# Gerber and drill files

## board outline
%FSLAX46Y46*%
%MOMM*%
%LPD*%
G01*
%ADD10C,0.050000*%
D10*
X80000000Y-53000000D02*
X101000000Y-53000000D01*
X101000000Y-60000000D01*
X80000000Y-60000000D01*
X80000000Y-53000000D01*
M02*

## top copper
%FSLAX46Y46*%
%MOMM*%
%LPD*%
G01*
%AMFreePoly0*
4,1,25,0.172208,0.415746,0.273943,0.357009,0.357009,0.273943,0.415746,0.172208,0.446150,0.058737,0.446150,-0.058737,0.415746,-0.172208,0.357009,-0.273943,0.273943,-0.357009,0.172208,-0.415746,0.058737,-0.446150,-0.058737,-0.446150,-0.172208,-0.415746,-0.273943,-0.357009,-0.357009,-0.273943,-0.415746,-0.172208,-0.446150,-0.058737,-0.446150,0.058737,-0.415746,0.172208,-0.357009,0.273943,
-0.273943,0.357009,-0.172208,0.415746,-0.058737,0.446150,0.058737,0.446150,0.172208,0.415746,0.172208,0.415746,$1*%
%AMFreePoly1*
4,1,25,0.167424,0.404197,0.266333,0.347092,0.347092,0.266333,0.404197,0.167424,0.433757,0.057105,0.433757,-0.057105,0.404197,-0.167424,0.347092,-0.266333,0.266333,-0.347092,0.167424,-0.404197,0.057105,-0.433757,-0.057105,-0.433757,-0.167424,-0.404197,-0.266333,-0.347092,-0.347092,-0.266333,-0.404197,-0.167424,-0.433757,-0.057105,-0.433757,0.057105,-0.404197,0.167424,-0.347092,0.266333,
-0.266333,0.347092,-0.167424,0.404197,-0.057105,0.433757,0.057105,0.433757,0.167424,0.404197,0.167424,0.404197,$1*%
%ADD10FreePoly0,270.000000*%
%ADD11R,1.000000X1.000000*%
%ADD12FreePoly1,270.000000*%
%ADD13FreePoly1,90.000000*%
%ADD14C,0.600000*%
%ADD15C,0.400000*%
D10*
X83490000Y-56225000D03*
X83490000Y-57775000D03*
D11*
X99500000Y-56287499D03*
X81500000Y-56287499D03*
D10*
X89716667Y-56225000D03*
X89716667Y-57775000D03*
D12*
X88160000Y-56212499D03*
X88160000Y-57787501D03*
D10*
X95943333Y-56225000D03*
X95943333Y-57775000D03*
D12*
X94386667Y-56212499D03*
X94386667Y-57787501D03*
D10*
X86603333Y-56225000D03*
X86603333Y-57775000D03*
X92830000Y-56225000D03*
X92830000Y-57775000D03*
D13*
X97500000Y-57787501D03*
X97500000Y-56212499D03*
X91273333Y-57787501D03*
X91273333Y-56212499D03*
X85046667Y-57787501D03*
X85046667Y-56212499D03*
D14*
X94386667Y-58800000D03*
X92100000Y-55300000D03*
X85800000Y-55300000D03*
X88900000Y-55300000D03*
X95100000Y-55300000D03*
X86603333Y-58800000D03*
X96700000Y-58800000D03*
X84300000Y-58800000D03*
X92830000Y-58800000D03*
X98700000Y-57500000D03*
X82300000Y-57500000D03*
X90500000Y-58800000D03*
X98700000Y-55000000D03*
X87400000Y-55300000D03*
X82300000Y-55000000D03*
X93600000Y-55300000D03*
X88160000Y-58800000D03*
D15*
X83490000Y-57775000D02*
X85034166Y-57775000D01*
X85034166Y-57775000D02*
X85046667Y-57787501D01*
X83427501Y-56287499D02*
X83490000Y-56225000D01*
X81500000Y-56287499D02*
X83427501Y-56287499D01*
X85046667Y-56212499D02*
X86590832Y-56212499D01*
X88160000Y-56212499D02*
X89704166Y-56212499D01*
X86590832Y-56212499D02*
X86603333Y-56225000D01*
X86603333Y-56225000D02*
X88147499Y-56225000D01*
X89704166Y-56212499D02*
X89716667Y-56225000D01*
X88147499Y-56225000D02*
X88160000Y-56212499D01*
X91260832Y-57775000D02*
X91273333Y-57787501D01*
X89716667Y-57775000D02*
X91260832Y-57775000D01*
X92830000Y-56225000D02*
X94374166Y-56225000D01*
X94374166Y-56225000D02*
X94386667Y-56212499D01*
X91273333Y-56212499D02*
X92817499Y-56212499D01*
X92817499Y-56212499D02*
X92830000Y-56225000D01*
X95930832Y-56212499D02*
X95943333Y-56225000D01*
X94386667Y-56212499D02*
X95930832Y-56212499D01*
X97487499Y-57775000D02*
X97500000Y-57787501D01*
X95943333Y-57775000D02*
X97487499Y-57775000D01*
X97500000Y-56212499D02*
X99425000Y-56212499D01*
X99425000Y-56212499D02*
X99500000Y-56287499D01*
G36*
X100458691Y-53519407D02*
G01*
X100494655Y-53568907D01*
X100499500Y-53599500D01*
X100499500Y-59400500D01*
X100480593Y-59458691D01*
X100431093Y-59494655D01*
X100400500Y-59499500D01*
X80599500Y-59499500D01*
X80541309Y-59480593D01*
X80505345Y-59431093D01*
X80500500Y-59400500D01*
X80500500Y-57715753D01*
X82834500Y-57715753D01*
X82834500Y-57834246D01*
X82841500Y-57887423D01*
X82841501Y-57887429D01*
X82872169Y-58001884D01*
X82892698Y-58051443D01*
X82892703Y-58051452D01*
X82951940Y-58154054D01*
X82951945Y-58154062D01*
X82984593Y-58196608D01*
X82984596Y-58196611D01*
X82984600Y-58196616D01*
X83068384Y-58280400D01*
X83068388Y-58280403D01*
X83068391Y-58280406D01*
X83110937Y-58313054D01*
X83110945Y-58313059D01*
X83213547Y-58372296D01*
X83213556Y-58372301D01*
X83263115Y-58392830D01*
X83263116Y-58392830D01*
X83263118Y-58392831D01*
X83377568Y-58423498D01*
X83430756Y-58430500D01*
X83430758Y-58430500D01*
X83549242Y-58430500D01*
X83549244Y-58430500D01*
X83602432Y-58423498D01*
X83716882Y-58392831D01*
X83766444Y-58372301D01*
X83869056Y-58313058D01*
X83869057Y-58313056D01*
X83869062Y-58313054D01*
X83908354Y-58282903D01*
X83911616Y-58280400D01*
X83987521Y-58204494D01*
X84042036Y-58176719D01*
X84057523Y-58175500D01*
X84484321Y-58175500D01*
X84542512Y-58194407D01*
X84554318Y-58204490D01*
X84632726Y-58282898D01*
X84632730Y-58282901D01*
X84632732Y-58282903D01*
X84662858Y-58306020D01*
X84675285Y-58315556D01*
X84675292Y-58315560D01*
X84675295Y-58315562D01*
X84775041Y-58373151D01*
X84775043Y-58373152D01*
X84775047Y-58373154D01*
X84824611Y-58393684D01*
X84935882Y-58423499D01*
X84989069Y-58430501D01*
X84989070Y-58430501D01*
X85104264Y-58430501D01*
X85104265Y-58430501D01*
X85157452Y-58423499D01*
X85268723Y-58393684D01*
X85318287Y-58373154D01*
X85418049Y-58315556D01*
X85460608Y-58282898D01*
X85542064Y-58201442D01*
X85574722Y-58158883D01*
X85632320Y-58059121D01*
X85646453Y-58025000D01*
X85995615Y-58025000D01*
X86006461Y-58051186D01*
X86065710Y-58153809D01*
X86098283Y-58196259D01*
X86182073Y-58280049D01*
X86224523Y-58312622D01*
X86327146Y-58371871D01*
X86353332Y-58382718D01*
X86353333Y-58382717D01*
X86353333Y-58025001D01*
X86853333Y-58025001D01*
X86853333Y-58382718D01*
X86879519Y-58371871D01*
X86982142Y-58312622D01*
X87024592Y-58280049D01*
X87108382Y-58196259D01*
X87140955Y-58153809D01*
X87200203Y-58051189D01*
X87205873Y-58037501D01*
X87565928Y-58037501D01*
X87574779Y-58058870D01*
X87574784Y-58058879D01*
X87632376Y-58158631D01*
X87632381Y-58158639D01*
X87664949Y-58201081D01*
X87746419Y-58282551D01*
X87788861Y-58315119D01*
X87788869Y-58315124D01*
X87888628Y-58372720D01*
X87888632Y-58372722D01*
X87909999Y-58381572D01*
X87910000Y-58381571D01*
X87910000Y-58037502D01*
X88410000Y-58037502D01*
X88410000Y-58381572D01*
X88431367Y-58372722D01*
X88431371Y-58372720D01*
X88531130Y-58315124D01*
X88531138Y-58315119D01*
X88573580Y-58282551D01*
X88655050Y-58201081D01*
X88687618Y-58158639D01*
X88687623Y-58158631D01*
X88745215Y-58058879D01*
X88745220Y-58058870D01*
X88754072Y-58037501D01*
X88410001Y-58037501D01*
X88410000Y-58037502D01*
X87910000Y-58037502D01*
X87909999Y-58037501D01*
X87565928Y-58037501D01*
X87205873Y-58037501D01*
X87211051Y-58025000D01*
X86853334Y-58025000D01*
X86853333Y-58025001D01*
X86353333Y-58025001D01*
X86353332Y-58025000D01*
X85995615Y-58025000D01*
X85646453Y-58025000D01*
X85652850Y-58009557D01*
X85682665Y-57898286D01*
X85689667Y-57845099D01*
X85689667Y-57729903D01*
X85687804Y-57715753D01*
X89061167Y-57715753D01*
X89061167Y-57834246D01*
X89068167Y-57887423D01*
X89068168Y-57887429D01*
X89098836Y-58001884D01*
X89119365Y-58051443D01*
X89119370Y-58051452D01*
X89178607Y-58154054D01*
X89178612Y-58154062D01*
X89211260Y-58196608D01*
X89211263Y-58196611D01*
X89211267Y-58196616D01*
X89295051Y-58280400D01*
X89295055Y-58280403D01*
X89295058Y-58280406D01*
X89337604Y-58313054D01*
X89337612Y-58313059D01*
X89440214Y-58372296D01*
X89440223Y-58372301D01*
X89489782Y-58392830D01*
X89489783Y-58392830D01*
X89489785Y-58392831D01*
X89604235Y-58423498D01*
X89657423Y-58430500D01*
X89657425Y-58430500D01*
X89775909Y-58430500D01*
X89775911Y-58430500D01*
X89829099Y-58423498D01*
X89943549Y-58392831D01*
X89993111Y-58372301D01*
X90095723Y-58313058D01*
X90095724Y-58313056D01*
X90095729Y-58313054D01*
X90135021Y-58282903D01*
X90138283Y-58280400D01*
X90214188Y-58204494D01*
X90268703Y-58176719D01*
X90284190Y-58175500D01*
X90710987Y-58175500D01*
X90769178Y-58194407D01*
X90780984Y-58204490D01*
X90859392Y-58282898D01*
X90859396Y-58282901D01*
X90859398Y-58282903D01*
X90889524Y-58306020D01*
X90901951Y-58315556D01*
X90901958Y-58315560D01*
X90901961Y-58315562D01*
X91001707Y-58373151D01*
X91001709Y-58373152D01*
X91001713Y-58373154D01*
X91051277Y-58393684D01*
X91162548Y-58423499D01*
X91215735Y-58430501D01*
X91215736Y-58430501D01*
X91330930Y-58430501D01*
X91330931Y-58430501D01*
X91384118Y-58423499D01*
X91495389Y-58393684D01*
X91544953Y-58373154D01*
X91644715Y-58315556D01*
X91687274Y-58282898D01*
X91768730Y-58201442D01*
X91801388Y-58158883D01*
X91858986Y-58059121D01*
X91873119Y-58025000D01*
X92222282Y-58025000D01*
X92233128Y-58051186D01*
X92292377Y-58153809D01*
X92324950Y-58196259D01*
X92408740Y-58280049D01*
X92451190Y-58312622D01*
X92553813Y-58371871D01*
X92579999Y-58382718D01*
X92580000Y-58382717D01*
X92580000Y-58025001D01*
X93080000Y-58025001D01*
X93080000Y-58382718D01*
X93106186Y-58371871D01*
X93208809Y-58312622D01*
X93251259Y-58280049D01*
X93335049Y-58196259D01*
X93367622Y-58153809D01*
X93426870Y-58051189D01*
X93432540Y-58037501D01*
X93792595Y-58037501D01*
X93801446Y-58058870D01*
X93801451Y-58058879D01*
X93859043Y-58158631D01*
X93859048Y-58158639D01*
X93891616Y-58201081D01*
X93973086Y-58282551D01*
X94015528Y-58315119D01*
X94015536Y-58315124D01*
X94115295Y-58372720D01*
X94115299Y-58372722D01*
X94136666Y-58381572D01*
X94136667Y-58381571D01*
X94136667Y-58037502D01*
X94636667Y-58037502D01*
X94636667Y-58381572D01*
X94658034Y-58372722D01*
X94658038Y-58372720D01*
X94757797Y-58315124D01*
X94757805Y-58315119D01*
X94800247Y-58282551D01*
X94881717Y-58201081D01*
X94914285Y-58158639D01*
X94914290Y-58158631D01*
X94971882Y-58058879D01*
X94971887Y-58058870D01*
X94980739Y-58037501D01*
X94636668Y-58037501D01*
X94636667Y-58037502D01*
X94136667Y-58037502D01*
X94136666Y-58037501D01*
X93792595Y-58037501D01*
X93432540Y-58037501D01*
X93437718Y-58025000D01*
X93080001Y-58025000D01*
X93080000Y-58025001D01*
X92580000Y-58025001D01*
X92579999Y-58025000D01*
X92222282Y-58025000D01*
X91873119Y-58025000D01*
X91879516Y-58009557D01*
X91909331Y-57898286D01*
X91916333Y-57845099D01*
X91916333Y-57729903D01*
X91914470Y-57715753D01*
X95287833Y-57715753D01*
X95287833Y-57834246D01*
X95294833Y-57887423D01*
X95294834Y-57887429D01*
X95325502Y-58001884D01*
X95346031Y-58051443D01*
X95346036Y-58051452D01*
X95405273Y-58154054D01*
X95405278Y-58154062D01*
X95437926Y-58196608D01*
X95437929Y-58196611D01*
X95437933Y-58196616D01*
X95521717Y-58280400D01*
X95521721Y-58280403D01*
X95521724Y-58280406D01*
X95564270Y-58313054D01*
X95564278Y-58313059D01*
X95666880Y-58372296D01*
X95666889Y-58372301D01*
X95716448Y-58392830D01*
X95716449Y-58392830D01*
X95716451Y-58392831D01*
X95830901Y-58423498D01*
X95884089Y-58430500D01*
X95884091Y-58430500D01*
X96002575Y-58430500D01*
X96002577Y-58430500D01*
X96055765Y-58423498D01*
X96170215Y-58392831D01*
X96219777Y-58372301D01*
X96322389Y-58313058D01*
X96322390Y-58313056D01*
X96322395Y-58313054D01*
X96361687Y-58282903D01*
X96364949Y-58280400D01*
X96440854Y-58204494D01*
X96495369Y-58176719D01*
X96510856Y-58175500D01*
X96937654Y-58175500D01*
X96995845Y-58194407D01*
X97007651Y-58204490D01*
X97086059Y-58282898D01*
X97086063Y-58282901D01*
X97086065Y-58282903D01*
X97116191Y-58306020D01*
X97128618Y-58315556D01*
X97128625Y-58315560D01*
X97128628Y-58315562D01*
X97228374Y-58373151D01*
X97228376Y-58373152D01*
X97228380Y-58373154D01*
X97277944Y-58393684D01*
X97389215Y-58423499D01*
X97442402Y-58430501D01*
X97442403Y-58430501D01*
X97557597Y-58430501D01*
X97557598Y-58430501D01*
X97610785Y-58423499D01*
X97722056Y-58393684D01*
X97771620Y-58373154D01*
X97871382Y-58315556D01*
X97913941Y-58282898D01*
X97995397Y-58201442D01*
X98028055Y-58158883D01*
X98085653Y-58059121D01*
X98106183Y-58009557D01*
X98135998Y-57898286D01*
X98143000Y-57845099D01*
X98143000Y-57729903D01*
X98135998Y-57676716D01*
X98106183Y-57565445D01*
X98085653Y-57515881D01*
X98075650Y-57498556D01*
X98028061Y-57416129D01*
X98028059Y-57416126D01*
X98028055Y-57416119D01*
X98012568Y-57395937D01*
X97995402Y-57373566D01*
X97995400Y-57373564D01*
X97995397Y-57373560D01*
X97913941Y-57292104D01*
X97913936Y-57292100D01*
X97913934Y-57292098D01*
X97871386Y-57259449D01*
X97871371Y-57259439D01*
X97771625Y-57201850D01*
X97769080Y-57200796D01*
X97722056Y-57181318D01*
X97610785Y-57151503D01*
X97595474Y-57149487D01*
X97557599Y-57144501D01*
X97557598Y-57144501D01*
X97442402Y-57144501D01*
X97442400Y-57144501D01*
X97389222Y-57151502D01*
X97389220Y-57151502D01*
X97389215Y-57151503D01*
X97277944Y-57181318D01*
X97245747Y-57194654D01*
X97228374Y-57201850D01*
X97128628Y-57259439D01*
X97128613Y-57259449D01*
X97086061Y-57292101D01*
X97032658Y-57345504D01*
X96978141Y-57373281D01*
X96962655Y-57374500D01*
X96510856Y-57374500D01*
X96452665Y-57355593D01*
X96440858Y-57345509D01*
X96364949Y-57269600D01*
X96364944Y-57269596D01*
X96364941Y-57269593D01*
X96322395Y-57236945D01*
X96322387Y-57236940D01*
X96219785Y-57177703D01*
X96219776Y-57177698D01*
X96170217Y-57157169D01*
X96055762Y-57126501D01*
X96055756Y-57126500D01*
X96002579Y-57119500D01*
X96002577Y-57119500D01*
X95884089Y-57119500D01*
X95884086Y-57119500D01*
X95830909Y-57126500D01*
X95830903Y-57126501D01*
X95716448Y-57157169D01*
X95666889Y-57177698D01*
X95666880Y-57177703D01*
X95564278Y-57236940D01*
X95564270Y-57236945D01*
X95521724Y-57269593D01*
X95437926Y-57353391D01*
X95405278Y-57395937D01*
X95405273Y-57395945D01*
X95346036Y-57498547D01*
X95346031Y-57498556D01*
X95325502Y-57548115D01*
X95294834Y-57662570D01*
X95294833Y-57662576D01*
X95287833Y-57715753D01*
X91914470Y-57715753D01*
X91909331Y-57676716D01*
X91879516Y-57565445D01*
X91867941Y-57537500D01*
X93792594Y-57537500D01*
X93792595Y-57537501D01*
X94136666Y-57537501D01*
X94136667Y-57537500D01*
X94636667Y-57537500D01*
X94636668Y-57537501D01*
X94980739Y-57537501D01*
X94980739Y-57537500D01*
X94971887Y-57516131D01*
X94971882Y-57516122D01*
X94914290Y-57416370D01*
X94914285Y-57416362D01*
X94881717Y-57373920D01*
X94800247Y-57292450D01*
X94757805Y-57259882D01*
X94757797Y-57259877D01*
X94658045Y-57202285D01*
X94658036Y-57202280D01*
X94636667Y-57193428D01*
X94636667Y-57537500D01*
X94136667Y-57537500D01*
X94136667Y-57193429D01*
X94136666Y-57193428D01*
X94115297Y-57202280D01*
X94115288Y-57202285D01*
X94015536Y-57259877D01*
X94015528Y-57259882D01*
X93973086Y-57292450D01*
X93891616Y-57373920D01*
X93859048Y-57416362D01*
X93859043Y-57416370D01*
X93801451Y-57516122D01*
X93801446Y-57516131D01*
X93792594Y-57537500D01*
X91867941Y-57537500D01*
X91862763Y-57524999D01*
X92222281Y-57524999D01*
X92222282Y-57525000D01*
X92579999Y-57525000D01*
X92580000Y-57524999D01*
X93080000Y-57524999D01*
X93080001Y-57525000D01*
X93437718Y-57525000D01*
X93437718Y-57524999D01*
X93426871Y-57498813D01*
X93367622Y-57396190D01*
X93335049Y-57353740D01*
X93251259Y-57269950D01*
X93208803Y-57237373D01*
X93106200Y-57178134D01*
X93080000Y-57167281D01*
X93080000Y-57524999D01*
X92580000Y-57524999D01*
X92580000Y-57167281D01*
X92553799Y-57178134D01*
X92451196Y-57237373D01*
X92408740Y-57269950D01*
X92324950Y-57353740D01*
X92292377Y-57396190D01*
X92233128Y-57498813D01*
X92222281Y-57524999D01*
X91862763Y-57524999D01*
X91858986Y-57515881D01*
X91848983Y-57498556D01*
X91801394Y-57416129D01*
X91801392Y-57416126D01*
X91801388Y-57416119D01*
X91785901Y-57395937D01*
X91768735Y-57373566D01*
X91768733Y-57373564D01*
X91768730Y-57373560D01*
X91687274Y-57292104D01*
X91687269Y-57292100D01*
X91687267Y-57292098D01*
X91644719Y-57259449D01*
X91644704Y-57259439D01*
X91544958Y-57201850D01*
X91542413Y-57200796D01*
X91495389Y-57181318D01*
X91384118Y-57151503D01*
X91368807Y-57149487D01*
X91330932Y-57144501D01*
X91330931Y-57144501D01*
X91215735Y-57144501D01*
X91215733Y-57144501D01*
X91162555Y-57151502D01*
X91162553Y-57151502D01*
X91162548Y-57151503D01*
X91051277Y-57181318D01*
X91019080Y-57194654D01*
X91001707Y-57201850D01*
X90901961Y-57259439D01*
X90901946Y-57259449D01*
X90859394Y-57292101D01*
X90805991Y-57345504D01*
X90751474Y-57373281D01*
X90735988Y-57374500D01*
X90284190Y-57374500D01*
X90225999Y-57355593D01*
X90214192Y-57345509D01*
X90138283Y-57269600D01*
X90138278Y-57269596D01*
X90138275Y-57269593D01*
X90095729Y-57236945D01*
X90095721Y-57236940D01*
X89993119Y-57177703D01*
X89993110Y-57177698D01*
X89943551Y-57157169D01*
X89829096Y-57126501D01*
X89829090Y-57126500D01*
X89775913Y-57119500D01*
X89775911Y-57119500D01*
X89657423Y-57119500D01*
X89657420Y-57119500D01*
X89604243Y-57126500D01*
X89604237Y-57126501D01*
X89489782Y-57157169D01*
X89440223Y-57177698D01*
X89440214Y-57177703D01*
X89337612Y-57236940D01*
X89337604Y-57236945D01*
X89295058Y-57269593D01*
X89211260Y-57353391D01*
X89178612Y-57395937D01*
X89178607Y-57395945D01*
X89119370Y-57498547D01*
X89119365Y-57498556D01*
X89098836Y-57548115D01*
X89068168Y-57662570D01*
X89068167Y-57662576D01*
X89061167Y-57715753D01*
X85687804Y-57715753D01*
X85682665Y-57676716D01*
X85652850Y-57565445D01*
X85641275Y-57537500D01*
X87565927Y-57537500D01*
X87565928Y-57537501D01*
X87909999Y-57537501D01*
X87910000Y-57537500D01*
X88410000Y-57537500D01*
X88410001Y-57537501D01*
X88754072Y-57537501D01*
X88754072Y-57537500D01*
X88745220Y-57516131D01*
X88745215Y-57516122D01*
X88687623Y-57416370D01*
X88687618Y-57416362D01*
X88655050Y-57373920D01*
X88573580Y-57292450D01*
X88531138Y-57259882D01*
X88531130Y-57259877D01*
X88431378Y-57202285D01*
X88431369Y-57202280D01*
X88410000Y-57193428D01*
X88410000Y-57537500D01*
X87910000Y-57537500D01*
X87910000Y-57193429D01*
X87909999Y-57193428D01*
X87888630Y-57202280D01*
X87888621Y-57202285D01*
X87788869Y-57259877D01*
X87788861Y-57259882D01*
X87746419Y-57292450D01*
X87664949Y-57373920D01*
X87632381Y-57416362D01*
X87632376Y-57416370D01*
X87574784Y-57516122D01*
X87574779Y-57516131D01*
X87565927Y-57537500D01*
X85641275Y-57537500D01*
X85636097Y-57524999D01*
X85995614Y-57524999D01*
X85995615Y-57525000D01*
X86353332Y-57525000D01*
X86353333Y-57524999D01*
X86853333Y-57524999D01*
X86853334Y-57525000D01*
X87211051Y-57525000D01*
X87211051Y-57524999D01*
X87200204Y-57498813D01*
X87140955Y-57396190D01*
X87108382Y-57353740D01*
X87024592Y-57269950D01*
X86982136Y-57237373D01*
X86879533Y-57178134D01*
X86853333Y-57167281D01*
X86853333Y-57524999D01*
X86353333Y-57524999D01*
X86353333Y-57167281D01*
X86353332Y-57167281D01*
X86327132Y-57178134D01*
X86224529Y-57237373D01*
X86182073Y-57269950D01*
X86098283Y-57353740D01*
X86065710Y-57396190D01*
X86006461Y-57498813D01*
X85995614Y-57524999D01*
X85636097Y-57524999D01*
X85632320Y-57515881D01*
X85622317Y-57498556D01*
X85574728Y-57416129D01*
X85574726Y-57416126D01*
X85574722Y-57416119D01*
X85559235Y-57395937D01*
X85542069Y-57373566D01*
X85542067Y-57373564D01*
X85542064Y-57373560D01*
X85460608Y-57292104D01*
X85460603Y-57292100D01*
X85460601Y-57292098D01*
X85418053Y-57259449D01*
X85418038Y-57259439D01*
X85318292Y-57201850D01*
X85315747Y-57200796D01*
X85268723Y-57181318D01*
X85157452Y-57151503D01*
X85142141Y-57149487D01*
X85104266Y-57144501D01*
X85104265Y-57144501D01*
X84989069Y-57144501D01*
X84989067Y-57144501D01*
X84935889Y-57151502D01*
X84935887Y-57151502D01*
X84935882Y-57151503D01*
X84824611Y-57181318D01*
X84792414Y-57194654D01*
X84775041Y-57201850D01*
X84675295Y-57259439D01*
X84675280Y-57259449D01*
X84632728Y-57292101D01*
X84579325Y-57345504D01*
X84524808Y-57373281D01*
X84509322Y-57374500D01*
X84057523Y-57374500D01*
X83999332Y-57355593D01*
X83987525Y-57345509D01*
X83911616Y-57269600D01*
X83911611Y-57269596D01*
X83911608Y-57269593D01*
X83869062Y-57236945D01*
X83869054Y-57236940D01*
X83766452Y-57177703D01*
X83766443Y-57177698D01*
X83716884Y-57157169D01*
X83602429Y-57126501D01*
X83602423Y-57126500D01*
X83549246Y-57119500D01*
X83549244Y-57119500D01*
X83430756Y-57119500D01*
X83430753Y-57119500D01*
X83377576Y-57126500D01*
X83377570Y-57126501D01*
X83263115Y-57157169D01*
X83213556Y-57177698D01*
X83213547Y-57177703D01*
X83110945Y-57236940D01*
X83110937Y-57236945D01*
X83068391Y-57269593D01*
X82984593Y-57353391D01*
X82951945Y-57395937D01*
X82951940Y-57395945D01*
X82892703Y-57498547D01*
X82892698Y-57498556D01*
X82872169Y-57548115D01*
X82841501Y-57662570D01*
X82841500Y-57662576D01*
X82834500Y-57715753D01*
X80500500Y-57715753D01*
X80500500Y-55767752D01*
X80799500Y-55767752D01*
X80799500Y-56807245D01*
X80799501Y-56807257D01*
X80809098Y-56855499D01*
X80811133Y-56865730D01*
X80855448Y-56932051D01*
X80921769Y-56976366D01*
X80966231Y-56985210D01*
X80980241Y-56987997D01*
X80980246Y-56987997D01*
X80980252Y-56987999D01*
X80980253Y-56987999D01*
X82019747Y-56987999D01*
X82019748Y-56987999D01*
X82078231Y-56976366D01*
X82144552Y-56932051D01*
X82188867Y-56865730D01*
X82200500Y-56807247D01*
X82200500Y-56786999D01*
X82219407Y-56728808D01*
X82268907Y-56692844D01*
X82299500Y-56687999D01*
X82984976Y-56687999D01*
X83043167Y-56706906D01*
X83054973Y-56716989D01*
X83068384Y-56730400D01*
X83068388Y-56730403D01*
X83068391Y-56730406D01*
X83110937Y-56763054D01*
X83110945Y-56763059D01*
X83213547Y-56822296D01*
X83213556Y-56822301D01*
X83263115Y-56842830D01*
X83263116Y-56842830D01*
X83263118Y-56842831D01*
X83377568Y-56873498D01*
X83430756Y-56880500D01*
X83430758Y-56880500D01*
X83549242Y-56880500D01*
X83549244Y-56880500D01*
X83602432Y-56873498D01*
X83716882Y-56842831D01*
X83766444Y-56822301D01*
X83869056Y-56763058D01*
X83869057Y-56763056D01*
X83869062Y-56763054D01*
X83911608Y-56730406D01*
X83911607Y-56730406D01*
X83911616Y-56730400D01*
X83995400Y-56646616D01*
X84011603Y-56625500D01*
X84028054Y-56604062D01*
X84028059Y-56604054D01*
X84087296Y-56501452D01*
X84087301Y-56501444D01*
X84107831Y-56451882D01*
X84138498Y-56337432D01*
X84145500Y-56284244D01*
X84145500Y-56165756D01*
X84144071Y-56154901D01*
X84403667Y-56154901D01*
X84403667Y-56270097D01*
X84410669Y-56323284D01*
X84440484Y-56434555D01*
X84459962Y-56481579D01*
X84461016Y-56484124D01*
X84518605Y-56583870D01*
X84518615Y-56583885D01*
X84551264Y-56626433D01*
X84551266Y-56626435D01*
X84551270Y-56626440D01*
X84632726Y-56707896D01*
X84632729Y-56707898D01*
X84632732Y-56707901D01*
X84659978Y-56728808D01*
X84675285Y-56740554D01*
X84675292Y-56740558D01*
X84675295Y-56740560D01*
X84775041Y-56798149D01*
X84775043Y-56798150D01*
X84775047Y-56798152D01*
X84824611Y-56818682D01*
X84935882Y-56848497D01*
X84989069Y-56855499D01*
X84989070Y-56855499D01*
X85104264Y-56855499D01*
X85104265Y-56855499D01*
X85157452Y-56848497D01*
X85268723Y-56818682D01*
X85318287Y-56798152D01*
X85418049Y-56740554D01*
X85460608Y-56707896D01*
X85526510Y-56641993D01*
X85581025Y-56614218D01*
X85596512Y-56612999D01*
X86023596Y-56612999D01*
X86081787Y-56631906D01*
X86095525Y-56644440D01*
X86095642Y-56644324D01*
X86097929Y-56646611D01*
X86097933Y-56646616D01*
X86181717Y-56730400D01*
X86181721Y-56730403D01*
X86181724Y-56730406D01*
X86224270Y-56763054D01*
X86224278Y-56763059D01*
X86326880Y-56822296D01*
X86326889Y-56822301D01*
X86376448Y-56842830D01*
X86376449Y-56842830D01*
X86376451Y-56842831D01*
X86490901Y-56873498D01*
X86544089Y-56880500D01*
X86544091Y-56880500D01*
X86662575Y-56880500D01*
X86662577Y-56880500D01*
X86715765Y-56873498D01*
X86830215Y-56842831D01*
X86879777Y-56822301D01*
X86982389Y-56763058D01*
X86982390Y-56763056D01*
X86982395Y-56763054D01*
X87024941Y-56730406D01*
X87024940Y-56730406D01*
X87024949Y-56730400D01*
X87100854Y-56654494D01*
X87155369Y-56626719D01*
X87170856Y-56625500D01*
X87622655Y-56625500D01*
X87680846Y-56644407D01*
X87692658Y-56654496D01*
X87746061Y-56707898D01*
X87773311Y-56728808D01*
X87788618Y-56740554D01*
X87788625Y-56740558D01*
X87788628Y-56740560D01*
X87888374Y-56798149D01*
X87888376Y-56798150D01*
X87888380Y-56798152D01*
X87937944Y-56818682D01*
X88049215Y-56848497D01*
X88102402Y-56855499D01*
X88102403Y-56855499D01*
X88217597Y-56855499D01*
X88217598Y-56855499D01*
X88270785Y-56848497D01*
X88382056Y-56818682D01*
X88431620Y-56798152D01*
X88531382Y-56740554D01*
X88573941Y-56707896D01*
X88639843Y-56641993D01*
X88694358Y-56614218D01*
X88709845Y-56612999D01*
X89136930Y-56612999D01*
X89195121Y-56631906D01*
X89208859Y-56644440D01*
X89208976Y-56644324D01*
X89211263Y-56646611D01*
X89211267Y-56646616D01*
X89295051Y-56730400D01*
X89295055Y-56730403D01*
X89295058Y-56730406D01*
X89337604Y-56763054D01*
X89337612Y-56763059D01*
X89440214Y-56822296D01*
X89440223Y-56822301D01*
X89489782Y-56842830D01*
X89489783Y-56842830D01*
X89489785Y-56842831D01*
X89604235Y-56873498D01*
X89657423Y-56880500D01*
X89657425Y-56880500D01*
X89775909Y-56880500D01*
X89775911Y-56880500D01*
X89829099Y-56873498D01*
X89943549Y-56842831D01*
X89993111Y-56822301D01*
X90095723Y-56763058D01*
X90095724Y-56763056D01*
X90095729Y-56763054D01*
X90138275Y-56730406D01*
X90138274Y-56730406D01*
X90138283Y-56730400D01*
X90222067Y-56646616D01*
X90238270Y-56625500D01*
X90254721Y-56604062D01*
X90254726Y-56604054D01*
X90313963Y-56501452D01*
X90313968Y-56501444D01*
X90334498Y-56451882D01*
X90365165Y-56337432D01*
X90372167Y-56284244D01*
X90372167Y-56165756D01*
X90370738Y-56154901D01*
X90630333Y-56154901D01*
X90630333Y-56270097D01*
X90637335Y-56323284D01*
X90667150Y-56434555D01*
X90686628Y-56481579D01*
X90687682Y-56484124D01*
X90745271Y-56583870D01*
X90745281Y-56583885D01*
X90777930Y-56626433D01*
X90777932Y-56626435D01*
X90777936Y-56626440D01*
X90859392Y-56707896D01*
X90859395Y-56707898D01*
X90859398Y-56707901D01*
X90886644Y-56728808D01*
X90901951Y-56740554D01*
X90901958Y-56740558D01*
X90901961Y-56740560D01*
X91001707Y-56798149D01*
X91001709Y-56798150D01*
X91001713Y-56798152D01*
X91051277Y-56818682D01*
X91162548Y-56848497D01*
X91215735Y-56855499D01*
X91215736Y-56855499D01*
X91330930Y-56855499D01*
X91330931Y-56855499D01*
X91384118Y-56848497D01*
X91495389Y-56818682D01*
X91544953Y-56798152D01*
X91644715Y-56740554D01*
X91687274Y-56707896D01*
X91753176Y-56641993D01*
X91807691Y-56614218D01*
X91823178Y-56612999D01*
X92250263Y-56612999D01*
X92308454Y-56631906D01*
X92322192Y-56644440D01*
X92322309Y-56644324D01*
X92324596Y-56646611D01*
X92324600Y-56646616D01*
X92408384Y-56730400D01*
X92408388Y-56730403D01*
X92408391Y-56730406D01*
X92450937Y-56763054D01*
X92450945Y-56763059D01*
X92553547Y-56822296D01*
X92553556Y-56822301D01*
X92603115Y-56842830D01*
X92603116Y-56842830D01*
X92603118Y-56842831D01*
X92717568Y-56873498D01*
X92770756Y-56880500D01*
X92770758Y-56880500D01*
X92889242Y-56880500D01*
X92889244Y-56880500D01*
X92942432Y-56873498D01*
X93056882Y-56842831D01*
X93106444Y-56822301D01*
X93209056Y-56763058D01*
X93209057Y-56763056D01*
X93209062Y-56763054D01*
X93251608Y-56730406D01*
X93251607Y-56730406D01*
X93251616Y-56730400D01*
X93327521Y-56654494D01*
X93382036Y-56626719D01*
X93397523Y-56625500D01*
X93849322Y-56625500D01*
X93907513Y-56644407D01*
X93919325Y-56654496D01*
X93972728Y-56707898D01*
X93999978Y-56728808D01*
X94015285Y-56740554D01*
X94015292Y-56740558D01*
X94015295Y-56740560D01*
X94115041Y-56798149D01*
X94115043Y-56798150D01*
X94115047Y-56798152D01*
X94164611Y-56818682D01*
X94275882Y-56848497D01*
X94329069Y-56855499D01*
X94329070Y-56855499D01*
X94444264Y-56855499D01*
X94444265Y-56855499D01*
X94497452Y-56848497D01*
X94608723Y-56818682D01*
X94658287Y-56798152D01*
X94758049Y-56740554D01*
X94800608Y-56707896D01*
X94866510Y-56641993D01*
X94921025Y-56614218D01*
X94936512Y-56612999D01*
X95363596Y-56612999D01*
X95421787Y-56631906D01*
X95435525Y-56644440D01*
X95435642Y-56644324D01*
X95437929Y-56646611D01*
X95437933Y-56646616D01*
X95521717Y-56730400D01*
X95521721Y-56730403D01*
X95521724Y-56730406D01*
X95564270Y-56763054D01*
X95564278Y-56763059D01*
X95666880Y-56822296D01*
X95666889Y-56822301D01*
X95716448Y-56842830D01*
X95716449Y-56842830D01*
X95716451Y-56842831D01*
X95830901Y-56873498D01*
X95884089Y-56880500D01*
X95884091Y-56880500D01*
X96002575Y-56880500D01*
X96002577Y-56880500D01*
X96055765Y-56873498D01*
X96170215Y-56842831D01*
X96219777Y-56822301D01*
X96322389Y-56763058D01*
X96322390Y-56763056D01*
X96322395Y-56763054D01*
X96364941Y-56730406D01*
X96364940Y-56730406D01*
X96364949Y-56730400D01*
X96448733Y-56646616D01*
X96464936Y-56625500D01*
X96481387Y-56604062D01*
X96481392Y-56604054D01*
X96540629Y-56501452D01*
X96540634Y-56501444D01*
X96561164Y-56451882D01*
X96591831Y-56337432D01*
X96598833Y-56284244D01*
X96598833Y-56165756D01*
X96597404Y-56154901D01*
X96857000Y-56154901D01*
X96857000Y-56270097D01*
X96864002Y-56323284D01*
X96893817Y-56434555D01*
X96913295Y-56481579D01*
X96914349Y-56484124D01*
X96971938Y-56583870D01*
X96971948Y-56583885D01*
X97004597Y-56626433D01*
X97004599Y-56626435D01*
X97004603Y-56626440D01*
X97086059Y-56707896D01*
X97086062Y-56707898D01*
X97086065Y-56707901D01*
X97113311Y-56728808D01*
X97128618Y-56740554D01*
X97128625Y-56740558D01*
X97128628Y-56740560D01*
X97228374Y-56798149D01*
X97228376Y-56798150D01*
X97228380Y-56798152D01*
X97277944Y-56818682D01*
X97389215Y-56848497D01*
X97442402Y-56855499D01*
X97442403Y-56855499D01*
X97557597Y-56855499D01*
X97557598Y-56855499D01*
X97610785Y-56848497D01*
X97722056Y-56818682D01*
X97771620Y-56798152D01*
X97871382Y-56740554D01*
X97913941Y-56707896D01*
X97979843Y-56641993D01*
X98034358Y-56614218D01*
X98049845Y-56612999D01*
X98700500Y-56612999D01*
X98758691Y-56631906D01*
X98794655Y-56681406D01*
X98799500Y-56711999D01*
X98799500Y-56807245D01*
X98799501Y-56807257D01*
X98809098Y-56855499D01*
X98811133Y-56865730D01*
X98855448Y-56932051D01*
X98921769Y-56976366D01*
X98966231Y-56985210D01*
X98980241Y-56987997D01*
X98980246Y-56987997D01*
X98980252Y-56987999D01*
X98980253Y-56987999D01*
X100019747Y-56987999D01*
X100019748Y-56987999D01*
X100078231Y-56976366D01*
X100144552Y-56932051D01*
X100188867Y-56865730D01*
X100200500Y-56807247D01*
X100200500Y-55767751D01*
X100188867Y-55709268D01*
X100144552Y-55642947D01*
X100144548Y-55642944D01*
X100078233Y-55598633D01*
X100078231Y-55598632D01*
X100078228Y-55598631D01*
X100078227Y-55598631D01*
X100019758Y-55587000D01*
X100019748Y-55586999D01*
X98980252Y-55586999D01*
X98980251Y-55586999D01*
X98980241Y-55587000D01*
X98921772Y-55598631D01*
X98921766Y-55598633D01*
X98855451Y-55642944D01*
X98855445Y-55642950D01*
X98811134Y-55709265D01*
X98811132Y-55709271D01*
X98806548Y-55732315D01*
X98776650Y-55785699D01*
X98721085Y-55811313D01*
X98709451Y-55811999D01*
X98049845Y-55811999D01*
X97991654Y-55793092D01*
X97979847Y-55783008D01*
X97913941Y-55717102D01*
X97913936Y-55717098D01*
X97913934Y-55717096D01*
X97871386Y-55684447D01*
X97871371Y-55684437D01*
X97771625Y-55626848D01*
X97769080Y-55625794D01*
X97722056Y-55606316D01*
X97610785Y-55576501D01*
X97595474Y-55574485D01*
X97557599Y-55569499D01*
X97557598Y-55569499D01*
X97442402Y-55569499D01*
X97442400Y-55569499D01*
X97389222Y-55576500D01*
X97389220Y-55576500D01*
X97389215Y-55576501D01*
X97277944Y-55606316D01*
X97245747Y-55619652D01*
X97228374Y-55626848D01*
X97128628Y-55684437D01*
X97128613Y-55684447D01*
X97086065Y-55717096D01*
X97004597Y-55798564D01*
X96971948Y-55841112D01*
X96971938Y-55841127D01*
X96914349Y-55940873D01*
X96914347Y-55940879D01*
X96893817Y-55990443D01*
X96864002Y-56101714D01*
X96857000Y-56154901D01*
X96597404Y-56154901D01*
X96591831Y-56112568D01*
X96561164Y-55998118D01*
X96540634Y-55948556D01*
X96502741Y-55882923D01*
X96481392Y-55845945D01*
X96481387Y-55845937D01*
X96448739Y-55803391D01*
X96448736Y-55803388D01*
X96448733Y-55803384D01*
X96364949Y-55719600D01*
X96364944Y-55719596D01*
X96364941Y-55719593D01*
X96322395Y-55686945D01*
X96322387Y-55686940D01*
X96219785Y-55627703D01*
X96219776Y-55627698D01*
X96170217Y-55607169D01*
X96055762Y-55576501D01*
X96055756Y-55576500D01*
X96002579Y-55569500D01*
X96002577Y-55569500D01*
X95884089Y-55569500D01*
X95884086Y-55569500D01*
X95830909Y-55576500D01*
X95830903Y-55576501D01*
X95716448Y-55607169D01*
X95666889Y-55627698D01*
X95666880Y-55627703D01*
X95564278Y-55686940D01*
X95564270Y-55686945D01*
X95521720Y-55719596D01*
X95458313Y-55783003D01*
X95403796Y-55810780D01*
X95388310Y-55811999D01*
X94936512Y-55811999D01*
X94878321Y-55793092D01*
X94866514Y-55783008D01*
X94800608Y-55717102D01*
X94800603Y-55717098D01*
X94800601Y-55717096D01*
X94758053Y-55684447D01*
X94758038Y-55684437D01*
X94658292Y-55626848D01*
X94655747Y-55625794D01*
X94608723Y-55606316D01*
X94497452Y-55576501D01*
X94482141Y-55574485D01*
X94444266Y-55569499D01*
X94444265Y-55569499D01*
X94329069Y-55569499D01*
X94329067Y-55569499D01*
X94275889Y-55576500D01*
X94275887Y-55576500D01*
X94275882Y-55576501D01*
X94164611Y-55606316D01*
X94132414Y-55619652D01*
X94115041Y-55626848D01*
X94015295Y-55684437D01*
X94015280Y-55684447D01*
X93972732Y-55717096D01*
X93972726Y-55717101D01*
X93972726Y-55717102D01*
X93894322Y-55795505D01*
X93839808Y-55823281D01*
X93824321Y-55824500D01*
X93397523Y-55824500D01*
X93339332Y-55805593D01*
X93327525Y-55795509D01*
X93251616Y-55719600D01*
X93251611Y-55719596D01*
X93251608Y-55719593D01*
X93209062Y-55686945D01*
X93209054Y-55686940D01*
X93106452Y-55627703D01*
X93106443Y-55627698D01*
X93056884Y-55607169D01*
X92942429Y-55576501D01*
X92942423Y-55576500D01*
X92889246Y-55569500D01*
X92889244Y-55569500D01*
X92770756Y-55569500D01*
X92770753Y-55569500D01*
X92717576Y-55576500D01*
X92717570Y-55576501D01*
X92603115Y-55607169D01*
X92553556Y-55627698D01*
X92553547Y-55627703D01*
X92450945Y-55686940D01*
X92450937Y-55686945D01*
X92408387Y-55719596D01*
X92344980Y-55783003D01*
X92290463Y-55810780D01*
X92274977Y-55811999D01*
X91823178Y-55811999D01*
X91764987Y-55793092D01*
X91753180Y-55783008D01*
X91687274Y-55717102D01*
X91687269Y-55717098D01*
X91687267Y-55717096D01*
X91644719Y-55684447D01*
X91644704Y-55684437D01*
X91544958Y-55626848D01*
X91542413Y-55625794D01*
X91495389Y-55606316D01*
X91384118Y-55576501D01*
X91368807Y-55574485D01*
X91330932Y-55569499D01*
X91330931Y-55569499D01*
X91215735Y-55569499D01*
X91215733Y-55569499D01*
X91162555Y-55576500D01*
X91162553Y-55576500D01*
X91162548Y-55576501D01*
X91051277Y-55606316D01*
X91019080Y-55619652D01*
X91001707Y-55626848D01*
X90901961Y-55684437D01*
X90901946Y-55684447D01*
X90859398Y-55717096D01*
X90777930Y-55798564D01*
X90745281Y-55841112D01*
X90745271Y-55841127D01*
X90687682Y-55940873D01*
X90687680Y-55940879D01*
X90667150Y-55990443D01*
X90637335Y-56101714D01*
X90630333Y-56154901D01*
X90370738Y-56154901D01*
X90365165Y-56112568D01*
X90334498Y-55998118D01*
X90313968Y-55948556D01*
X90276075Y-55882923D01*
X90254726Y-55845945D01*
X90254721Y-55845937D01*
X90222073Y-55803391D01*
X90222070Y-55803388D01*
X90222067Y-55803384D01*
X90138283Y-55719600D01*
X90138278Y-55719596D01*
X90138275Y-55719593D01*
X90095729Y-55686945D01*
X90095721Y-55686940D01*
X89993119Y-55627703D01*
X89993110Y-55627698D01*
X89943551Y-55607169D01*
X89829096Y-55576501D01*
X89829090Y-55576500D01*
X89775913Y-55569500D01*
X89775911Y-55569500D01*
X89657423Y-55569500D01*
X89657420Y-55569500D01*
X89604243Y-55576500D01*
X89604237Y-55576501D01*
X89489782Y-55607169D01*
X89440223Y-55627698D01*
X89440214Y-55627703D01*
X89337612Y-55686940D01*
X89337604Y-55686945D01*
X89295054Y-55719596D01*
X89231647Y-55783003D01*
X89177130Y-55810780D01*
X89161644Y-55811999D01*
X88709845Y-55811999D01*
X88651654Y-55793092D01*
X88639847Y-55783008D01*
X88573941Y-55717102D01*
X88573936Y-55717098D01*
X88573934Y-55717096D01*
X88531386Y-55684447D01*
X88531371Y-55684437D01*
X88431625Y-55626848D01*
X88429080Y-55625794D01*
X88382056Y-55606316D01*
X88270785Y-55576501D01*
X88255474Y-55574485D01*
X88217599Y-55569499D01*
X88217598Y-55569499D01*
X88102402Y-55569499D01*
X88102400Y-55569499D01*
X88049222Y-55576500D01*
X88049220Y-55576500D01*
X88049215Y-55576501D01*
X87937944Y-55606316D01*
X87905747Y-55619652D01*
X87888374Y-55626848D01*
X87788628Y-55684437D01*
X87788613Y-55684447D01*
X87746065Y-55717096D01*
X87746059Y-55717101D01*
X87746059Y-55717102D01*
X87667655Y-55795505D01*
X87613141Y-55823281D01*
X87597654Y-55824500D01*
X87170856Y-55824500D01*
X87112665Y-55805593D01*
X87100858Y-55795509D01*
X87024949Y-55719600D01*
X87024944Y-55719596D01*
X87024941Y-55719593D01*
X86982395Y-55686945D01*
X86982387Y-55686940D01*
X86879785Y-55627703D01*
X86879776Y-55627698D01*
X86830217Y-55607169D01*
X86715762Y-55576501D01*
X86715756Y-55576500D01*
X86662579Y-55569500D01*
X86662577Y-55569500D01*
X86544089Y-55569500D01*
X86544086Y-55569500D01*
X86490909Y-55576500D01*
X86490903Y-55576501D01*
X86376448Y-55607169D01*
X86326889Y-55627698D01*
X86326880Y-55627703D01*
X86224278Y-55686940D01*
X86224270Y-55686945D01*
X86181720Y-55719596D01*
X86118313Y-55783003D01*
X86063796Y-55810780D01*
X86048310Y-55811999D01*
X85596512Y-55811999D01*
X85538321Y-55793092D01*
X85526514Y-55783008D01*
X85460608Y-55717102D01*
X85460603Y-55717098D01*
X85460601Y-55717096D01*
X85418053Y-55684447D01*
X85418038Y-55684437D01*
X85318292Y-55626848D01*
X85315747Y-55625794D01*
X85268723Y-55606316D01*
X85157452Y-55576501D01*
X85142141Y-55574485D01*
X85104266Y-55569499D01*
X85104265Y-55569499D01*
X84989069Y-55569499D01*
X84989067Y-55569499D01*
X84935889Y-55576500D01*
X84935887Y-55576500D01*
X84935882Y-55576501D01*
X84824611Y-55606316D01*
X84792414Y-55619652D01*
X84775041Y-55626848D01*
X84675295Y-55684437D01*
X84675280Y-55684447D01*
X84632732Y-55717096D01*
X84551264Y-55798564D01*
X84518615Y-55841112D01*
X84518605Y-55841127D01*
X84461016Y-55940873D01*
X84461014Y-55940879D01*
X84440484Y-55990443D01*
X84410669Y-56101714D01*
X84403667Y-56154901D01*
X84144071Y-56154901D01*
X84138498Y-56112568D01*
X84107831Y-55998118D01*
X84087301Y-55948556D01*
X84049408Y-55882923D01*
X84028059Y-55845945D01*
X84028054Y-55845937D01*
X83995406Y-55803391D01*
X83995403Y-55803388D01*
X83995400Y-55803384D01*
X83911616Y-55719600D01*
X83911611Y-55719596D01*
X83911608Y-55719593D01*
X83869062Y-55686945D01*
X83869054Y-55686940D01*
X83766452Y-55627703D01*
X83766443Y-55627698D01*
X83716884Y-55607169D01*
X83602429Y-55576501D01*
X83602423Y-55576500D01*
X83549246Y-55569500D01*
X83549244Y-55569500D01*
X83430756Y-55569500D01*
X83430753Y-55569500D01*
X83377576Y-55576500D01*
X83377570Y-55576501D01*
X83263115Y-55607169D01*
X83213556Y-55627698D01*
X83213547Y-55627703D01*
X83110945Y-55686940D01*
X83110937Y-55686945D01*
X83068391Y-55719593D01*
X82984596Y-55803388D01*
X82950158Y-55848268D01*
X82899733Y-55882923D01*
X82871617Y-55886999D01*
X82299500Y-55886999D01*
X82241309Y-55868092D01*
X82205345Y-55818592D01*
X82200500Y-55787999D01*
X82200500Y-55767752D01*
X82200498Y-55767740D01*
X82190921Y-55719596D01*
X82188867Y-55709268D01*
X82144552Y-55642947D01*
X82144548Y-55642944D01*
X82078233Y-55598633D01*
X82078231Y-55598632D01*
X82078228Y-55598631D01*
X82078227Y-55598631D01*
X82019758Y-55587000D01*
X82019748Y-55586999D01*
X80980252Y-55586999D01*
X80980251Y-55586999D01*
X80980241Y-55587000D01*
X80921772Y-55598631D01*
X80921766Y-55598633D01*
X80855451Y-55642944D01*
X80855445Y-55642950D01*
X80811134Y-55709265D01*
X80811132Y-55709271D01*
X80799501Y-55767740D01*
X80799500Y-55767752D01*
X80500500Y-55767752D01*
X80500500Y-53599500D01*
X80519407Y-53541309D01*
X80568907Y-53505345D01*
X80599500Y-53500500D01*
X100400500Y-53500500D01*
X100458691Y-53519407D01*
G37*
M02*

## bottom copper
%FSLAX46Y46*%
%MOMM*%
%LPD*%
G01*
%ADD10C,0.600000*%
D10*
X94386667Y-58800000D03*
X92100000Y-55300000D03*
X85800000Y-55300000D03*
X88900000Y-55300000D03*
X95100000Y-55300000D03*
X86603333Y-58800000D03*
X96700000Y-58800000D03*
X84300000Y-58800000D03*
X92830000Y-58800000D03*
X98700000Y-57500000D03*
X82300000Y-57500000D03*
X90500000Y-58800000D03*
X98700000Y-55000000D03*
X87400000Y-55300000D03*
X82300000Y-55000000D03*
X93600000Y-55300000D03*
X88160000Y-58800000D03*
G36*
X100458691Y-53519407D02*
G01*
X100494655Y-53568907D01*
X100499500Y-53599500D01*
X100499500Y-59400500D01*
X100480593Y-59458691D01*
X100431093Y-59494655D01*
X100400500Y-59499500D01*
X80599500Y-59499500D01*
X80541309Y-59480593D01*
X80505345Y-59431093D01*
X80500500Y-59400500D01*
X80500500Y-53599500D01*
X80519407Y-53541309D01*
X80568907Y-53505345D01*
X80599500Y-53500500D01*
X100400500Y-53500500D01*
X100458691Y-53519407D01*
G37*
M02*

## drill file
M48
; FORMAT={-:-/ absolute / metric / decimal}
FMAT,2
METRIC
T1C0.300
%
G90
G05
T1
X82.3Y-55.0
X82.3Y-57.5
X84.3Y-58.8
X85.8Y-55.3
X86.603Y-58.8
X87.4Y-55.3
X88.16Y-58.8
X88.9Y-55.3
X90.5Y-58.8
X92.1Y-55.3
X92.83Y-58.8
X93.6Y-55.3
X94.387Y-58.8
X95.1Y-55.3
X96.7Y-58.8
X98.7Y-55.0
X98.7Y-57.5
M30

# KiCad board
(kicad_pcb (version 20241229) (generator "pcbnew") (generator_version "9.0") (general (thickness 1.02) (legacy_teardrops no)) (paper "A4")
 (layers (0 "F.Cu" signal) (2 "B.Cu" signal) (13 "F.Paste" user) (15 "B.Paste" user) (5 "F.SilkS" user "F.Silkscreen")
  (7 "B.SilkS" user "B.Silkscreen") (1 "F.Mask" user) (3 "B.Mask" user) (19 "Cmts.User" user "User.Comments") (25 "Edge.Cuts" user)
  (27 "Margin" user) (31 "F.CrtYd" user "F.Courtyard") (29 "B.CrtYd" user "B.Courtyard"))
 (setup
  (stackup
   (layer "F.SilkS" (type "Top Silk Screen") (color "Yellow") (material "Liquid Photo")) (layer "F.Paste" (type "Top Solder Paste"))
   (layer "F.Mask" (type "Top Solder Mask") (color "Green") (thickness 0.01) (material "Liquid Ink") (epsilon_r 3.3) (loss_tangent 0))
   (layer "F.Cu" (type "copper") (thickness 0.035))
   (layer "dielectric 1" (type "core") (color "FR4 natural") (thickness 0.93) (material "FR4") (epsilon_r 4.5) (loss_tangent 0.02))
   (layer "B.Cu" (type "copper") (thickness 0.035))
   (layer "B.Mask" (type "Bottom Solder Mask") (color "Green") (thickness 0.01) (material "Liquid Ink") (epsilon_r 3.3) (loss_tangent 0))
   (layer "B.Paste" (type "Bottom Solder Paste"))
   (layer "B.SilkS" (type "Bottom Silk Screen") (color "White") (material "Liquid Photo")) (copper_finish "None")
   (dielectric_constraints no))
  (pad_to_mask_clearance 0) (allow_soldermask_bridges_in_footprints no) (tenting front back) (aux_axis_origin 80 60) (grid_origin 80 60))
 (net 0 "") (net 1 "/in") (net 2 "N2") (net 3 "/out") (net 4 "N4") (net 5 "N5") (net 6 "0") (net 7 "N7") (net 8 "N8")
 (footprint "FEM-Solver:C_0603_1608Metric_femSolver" (layer "F.Cu") (at 83.49 57 -90)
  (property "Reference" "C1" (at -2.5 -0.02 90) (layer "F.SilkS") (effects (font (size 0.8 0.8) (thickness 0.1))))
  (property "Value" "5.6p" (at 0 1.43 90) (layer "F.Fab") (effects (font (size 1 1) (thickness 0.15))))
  (pad "1" smd custom (at -0.775 0 270) (size 0.9 0.9) (layers "F.Cu" "F.Mask" "F.Paste") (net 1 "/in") (thermal_bridge_angle 90)
   (options (clearance outline) (anchor circle)) (primitives))
  (pad "2" smd custom (at 0.775 0 270) (size 0.9 0.9) (layers "F.Cu" "F.Mask" "F.Paste") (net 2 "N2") (thermal_bridge_angle 90)
   (options (clearance outline) (anchor circle)) (primitives)))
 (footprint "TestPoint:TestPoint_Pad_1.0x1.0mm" (layer "F.Cu") (at 99.5 56.287499)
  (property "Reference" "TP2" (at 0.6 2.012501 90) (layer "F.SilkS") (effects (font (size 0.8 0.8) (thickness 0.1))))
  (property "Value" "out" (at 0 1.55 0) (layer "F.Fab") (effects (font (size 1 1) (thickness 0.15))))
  (pad "1" smd rect (at 0 0) (size 1 1) (layers "F.Cu" "F.Mask") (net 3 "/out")))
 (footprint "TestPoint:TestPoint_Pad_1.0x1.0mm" (layer "F.Cu") (at 81.5 56.287499)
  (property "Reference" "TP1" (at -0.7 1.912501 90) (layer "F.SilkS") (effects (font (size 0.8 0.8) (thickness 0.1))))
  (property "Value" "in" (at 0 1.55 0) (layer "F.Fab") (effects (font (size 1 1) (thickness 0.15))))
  (pad "1" smd rect (at 0 0) (size 1 1) (layers "F.Cu" "F.Mask") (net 1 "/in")))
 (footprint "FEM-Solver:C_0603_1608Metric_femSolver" (layer "F.Cu") (at 89.716667 57 -90)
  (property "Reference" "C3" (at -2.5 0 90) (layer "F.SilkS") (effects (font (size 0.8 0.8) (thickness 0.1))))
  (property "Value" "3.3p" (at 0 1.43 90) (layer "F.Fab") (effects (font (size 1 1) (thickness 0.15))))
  (pad "1" smd custom (at -0.775 0 270) (size 0.9 0.9) (layers "F.Cu" "F.Mask" "F.Paste") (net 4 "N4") (thermal_bridge_angle 90)
   (options (clearance outline) (anchor circle)) (primitives))
  (pad "2" smd custom (at 0.775 0 270) (size 0.9 0.9) (layers "F.Cu" "F.Mask" "F.Paste") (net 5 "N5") (thermal_bridge_angle 90)
   (options (clearance outline) (anchor circle)) (primitives)))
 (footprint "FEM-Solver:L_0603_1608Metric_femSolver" (layer "F.Cu") (at 88.16 57 -90)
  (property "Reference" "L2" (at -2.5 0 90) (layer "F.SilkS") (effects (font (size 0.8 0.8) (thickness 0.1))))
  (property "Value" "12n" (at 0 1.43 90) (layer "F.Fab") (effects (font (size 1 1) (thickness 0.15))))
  (pad "1" smd custom (at -0.787501 0 270) (size 0.875 0.875) (layers "F.Cu" "F.Mask" "F.Paste") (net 4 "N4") (thermal_bridge_angle 90)
   (options (clearance outline) (anchor circle)) (primitives))
  (pad "2" smd custom (at 0.787501 0 270) (size 0.875 0.875) (layers "F.Cu" "F.Mask" "F.Paste") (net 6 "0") (thermal_bridge_angle 90)
   (options (clearance outline) (anchor circle)) (primitives)))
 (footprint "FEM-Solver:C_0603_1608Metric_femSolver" (layer "F.Cu") (at 95.943333 57 -90)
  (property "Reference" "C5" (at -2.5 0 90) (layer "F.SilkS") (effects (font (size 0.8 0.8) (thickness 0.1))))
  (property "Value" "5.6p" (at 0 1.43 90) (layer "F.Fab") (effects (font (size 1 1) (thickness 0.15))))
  (pad "1" smd custom (at -0.775 0 270) (size 0.9 0.9) (layers "F.Cu" "F.Mask" "F.Paste") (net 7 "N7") (thermal_bridge_angle 90)
   (options (clearance outline) (anchor circle)) (primitives))
  (pad "2" smd custom (at 0.775 0 270) (size 0.9 0.9) (layers "F.Cu" "F.Mask" "F.Paste") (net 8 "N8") (thermal_bridge_angle 90)
   (options (clearance outline) (anchor circle)) (primitives)))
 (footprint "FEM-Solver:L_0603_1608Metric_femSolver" (layer "F.Cu") (at 94.386667 57 -90)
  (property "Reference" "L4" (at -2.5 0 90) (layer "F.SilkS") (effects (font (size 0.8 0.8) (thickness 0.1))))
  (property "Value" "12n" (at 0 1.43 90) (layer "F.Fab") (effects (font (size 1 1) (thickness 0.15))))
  (pad "1" smd custom (at -0.787501 0 270) (size 0.875 0.875) (layers "F.Cu" "F.Mask" "F.Paste") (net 7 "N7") (thermal_bridge_angle 90)
   (options (clearance outline) (anchor circle)) (primitives))
  (pad "2" smd custom (at 0.787501 0 270) (size 0.875 0.875) (layers "F.Cu" "F.Mask" "F.Paste") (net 6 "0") (thermal_bridge_angle 90)
   (options (clearance outline) (anchor circle)) (primitives)))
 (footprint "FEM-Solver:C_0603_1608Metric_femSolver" (layer "F.Cu") (at 86.603333 57 -90)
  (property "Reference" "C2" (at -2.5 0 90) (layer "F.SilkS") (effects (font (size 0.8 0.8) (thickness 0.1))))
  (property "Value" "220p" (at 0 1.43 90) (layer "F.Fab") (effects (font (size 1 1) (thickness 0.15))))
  (pad "1" smd custom (at -0.775 0 270) (size 0.9 0.9) (layers "F.Cu" "F.Mask" "F.Paste") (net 4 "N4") (thermal_bridge_angle 90)
   (options (clearance outline) (anchor circle)) (primitives))
  (pad "2" smd custom (at 0.775 0 270) (size 0.9 0.9) (layers "F.Cu" "F.Mask" "F.Paste") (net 6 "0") (thermal_bridge_angle 90)
   (options (clearance outline) (anchor circle)) (primitives)))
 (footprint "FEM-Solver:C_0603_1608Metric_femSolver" (layer "F.Cu") (at 92.83 57 -90)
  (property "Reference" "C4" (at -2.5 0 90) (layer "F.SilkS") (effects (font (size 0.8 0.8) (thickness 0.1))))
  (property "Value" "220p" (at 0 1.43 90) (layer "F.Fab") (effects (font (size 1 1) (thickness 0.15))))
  (pad "1" smd custom (at -0.775 0 270) (size 0.9 0.9) (layers "F.Cu" "F.Mask" "F.Paste") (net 7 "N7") (thermal_bridge_angle 90)
   (options (clearance outline) (anchor circle)) (primitives))
  (pad "2" smd custom (at 0.775 0 270) (size 0.9 0.9) (layers "F.Cu" "F.Mask" "F.Paste") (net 6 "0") (thermal_bridge_angle 90)
   (options (clearance outline) (anchor circle)) (primitives)))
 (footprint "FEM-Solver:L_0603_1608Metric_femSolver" (layer "F.Cu") (at 97.5 57 90)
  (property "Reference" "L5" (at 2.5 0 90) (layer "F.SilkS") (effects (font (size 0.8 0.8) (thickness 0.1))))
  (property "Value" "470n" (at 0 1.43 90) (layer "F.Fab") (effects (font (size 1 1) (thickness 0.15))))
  (pad "1" smd custom (at -0.787501 0 90) (size 0.875 0.875) (layers "F.Cu" "F.Mask" "F.Paste") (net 8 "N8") (thermal_bridge_angle 90)
   (options (clearance outline) (anchor circle)) (primitives))
  (pad "2" smd custom (at 0.787501 0 90) (size 0.875 0.875) (layers "F.Cu" "F.Mask" "F.Paste") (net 3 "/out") (thermal_bridge_angle 90)
   (options (clearance outline) (anchor circle)) (primitives)))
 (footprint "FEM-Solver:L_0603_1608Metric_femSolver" (layer "F.Cu") (at 91.273333 57 90)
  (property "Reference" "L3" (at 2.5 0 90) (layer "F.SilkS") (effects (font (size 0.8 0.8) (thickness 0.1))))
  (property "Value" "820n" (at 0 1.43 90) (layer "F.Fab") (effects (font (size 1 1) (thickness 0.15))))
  (pad "1" smd custom (at -0.787501 0 90) (size 0.875 0.875) (layers "F.Cu" "F.Mask" "F.Paste") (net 5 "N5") (thermal_bridge_angle 90)
   (options (clearance outline) (anchor circle)) (primitives))
  (pad "2" smd custom (at 0.787501 0 90) (size 0.875 0.875) (layers "F.Cu" "F.Mask" "F.Paste") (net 7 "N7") (thermal_bridge_angle 90)
   (options (clearance outline) (anchor circle)) (primitives)))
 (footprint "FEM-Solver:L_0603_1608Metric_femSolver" (layer "F.Cu") (at 85.046667 57 90)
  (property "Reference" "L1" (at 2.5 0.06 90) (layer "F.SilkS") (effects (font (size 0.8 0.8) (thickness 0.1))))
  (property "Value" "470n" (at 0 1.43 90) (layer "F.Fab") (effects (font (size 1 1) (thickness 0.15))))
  (pad "1" smd custom (at -0.787501 0 90) (size 0.875 0.875) (layers "F.Cu" "F.Mask" "F.Paste") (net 2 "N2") (thermal_bridge_angle 90)
   (options (clearance outline) (anchor circle)) (primitives))
  (pad "2" smd custom (at 0.787501 0 90) (size 0.875 0.875) (layers "F.Cu" "F.Mask" "F.Paste") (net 4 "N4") (thermal_bridge_angle 90)
   (options (clearance outline) (anchor circle)) (primitives)))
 (gr_rect (start 80 53) (end 101 60) (stroke (width 0.05) (type default)) (fill no) (layer "Edge.Cuts"))
 (segment (start 83.49 57.775) (end 85.034166 57.775) (width 0.4) (layer "F.Cu") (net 2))
 (segment (start 85.034166 57.775) (end 85.046667 57.787501) (width 0.4) (layer "F.Cu") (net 2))
 (segment (start 83.427501 56.287499) (end 83.49 56.225) (width 0.4) (layer "F.Cu") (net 1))
 (segment (start 81.5 56.287499) (end 83.427501 56.287499) (width 0.4) (layer "F.Cu") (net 1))
 (via (at 94.386667 58.8) (size 0.6) (drill 0.3) (layers "F.Cu" "B.Cu") (free yes) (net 6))
 (via (at 92.1 55.3) (size 0.6) (drill 0.3) (layers "F.Cu" "B.Cu") (free yes) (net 6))
 (via (at 85.8 55.3) (size 0.6) (drill 0.3) (layers "F.Cu" "B.Cu") (free yes) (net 6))
 (via (at 88.9 55.3) (size 0.6) (drill 0.3) (layers "F.Cu" "B.Cu") (free yes) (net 6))
 (via (at 95.1 55.3) (size 0.6) (drill 0.3) (layers "F.Cu" "B.Cu") (free yes) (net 6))
 (via (at 86.603333 58.8) (size 0.6) (drill 0.3) (layers "F.Cu" "B.Cu") (free yes) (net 6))
 (via (at 96.7 58.8) (size 0.6) (drill 0.3) (layers "F.Cu" "B.Cu") (free yes) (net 6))
 (via (at 84.3 58.8) (size 0.6) (drill 0.3) (layers "F.Cu" "B.Cu") (free yes) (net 6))
 (via (at 92.83 58.8) (size 0.6) (drill 0.3) (layers "F.Cu" "B.Cu") (free yes) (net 6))
 (via (at 98.7 57.5) (size 0.6) (drill 0.3) (layers "F.Cu" "B.Cu") (free yes) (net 6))
 (via (at 82.3 57.5) (size 0.6) (drill 0.3) (layers "F.Cu" "B.Cu") (free yes) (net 6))
 (via (at 90.5 58.8) (size 0.6) (drill 0.3) (layers "F.Cu" "B.Cu") (free yes) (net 6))
 (via (at 98.7 55) (size 0.6) (drill 0.3) (layers "F.Cu" "B.Cu") (free yes) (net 6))
 (via (at 87.4 55.3) (size 0.6) (drill 0.3) (layers "F.Cu" "B.Cu") (free yes) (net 6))
 (via (at 82.3 55) (size 0.6) (drill 0.3) (layers "F.Cu" "B.Cu") (free yes) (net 6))
 (via (at 93.6 55.3) (size 0.6) (drill 0.3) (layers "F.Cu" "B.Cu") (free yes) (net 6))
 (via (at 88.16 58.8) (size 0.6) (drill 0.3) (layers "F.Cu" "B.Cu") (free yes) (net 6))
 (segment (start 85.046667 56.212499) (end 86.590832 56.212499) (width 0.4) (layer "F.Cu") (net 4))
 (segment (start 88.16 56.212499) (end 89.704166 56.212499) (width 0.4) (layer "F.Cu") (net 4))
 (segment (start 86.590832 56.212499) (end 86.603333 56.225) (width 0.4) (layer "F.Cu") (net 4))
 (segment (start 86.603333 56.225) (end 88.147499 56.225) (width 0.4) (layer "F.Cu") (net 4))
 (segment (start 89.704166 56.212499) (end 89.716667 56.225) (width 0.4) (layer "F.Cu") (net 4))
 (segment (start 88.147499 56.225) (end 88.16 56.212499) (width 0.4) (layer "F.Cu") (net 4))
 (segment (start 91.260832 57.775) (end 91.273333 57.787501) (width 0.4) (layer "F.Cu") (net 5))
 (segment (start 89.716667 57.775) (end 91.260832 57.775) (width 0.4) (layer "F.Cu") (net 5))
 (segment (start 92.83 56.225) (end 94.374166 56.225) (width 0.4) (layer "F.Cu") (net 7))
 (segment (start 94.374166 56.225) (end 94.386667 56.212499) (width 0.4) (layer "F.Cu") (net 7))
 (segment (start 91.273333 56.212499) (end 92.817499 56.212499) (width 0.4) (layer "F.Cu") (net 7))
 (segment (start 92.817499 56.212499) (end 92.83 56.225) (width 0.4) (layer "F.Cu") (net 7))
 (segment (start 95.930832 56.212499) (end 95.943333 56.225) (width 0.4) (layer "F.Cu") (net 7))
 (segment (start 94.386667 56.212499) (end 95.930832 56.212499) (width 0.4) (layer "F.Cu") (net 7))
 (segment (start 97.487499 57.775) (end 97.5 57.787501) (width 0.4) (layer "F.Cu") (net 8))
 (segment (start 95.943333 57.775) (end 97.487499 57.775) (width 0.4) (layer "F.Cu") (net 8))
 (segment (start 97.5 56.212499) (end 99.425 56.212499) (width 0.4) (layer "F.Cu") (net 3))
 (segment (start 99.425 56.212499) (end 99.5 56.287499) (width 0.4) (layer "F.Cu") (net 3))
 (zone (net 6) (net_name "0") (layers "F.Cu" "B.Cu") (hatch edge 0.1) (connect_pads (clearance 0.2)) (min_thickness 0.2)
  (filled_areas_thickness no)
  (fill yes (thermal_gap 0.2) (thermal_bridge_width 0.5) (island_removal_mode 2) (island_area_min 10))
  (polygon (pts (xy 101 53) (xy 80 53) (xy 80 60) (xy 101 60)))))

